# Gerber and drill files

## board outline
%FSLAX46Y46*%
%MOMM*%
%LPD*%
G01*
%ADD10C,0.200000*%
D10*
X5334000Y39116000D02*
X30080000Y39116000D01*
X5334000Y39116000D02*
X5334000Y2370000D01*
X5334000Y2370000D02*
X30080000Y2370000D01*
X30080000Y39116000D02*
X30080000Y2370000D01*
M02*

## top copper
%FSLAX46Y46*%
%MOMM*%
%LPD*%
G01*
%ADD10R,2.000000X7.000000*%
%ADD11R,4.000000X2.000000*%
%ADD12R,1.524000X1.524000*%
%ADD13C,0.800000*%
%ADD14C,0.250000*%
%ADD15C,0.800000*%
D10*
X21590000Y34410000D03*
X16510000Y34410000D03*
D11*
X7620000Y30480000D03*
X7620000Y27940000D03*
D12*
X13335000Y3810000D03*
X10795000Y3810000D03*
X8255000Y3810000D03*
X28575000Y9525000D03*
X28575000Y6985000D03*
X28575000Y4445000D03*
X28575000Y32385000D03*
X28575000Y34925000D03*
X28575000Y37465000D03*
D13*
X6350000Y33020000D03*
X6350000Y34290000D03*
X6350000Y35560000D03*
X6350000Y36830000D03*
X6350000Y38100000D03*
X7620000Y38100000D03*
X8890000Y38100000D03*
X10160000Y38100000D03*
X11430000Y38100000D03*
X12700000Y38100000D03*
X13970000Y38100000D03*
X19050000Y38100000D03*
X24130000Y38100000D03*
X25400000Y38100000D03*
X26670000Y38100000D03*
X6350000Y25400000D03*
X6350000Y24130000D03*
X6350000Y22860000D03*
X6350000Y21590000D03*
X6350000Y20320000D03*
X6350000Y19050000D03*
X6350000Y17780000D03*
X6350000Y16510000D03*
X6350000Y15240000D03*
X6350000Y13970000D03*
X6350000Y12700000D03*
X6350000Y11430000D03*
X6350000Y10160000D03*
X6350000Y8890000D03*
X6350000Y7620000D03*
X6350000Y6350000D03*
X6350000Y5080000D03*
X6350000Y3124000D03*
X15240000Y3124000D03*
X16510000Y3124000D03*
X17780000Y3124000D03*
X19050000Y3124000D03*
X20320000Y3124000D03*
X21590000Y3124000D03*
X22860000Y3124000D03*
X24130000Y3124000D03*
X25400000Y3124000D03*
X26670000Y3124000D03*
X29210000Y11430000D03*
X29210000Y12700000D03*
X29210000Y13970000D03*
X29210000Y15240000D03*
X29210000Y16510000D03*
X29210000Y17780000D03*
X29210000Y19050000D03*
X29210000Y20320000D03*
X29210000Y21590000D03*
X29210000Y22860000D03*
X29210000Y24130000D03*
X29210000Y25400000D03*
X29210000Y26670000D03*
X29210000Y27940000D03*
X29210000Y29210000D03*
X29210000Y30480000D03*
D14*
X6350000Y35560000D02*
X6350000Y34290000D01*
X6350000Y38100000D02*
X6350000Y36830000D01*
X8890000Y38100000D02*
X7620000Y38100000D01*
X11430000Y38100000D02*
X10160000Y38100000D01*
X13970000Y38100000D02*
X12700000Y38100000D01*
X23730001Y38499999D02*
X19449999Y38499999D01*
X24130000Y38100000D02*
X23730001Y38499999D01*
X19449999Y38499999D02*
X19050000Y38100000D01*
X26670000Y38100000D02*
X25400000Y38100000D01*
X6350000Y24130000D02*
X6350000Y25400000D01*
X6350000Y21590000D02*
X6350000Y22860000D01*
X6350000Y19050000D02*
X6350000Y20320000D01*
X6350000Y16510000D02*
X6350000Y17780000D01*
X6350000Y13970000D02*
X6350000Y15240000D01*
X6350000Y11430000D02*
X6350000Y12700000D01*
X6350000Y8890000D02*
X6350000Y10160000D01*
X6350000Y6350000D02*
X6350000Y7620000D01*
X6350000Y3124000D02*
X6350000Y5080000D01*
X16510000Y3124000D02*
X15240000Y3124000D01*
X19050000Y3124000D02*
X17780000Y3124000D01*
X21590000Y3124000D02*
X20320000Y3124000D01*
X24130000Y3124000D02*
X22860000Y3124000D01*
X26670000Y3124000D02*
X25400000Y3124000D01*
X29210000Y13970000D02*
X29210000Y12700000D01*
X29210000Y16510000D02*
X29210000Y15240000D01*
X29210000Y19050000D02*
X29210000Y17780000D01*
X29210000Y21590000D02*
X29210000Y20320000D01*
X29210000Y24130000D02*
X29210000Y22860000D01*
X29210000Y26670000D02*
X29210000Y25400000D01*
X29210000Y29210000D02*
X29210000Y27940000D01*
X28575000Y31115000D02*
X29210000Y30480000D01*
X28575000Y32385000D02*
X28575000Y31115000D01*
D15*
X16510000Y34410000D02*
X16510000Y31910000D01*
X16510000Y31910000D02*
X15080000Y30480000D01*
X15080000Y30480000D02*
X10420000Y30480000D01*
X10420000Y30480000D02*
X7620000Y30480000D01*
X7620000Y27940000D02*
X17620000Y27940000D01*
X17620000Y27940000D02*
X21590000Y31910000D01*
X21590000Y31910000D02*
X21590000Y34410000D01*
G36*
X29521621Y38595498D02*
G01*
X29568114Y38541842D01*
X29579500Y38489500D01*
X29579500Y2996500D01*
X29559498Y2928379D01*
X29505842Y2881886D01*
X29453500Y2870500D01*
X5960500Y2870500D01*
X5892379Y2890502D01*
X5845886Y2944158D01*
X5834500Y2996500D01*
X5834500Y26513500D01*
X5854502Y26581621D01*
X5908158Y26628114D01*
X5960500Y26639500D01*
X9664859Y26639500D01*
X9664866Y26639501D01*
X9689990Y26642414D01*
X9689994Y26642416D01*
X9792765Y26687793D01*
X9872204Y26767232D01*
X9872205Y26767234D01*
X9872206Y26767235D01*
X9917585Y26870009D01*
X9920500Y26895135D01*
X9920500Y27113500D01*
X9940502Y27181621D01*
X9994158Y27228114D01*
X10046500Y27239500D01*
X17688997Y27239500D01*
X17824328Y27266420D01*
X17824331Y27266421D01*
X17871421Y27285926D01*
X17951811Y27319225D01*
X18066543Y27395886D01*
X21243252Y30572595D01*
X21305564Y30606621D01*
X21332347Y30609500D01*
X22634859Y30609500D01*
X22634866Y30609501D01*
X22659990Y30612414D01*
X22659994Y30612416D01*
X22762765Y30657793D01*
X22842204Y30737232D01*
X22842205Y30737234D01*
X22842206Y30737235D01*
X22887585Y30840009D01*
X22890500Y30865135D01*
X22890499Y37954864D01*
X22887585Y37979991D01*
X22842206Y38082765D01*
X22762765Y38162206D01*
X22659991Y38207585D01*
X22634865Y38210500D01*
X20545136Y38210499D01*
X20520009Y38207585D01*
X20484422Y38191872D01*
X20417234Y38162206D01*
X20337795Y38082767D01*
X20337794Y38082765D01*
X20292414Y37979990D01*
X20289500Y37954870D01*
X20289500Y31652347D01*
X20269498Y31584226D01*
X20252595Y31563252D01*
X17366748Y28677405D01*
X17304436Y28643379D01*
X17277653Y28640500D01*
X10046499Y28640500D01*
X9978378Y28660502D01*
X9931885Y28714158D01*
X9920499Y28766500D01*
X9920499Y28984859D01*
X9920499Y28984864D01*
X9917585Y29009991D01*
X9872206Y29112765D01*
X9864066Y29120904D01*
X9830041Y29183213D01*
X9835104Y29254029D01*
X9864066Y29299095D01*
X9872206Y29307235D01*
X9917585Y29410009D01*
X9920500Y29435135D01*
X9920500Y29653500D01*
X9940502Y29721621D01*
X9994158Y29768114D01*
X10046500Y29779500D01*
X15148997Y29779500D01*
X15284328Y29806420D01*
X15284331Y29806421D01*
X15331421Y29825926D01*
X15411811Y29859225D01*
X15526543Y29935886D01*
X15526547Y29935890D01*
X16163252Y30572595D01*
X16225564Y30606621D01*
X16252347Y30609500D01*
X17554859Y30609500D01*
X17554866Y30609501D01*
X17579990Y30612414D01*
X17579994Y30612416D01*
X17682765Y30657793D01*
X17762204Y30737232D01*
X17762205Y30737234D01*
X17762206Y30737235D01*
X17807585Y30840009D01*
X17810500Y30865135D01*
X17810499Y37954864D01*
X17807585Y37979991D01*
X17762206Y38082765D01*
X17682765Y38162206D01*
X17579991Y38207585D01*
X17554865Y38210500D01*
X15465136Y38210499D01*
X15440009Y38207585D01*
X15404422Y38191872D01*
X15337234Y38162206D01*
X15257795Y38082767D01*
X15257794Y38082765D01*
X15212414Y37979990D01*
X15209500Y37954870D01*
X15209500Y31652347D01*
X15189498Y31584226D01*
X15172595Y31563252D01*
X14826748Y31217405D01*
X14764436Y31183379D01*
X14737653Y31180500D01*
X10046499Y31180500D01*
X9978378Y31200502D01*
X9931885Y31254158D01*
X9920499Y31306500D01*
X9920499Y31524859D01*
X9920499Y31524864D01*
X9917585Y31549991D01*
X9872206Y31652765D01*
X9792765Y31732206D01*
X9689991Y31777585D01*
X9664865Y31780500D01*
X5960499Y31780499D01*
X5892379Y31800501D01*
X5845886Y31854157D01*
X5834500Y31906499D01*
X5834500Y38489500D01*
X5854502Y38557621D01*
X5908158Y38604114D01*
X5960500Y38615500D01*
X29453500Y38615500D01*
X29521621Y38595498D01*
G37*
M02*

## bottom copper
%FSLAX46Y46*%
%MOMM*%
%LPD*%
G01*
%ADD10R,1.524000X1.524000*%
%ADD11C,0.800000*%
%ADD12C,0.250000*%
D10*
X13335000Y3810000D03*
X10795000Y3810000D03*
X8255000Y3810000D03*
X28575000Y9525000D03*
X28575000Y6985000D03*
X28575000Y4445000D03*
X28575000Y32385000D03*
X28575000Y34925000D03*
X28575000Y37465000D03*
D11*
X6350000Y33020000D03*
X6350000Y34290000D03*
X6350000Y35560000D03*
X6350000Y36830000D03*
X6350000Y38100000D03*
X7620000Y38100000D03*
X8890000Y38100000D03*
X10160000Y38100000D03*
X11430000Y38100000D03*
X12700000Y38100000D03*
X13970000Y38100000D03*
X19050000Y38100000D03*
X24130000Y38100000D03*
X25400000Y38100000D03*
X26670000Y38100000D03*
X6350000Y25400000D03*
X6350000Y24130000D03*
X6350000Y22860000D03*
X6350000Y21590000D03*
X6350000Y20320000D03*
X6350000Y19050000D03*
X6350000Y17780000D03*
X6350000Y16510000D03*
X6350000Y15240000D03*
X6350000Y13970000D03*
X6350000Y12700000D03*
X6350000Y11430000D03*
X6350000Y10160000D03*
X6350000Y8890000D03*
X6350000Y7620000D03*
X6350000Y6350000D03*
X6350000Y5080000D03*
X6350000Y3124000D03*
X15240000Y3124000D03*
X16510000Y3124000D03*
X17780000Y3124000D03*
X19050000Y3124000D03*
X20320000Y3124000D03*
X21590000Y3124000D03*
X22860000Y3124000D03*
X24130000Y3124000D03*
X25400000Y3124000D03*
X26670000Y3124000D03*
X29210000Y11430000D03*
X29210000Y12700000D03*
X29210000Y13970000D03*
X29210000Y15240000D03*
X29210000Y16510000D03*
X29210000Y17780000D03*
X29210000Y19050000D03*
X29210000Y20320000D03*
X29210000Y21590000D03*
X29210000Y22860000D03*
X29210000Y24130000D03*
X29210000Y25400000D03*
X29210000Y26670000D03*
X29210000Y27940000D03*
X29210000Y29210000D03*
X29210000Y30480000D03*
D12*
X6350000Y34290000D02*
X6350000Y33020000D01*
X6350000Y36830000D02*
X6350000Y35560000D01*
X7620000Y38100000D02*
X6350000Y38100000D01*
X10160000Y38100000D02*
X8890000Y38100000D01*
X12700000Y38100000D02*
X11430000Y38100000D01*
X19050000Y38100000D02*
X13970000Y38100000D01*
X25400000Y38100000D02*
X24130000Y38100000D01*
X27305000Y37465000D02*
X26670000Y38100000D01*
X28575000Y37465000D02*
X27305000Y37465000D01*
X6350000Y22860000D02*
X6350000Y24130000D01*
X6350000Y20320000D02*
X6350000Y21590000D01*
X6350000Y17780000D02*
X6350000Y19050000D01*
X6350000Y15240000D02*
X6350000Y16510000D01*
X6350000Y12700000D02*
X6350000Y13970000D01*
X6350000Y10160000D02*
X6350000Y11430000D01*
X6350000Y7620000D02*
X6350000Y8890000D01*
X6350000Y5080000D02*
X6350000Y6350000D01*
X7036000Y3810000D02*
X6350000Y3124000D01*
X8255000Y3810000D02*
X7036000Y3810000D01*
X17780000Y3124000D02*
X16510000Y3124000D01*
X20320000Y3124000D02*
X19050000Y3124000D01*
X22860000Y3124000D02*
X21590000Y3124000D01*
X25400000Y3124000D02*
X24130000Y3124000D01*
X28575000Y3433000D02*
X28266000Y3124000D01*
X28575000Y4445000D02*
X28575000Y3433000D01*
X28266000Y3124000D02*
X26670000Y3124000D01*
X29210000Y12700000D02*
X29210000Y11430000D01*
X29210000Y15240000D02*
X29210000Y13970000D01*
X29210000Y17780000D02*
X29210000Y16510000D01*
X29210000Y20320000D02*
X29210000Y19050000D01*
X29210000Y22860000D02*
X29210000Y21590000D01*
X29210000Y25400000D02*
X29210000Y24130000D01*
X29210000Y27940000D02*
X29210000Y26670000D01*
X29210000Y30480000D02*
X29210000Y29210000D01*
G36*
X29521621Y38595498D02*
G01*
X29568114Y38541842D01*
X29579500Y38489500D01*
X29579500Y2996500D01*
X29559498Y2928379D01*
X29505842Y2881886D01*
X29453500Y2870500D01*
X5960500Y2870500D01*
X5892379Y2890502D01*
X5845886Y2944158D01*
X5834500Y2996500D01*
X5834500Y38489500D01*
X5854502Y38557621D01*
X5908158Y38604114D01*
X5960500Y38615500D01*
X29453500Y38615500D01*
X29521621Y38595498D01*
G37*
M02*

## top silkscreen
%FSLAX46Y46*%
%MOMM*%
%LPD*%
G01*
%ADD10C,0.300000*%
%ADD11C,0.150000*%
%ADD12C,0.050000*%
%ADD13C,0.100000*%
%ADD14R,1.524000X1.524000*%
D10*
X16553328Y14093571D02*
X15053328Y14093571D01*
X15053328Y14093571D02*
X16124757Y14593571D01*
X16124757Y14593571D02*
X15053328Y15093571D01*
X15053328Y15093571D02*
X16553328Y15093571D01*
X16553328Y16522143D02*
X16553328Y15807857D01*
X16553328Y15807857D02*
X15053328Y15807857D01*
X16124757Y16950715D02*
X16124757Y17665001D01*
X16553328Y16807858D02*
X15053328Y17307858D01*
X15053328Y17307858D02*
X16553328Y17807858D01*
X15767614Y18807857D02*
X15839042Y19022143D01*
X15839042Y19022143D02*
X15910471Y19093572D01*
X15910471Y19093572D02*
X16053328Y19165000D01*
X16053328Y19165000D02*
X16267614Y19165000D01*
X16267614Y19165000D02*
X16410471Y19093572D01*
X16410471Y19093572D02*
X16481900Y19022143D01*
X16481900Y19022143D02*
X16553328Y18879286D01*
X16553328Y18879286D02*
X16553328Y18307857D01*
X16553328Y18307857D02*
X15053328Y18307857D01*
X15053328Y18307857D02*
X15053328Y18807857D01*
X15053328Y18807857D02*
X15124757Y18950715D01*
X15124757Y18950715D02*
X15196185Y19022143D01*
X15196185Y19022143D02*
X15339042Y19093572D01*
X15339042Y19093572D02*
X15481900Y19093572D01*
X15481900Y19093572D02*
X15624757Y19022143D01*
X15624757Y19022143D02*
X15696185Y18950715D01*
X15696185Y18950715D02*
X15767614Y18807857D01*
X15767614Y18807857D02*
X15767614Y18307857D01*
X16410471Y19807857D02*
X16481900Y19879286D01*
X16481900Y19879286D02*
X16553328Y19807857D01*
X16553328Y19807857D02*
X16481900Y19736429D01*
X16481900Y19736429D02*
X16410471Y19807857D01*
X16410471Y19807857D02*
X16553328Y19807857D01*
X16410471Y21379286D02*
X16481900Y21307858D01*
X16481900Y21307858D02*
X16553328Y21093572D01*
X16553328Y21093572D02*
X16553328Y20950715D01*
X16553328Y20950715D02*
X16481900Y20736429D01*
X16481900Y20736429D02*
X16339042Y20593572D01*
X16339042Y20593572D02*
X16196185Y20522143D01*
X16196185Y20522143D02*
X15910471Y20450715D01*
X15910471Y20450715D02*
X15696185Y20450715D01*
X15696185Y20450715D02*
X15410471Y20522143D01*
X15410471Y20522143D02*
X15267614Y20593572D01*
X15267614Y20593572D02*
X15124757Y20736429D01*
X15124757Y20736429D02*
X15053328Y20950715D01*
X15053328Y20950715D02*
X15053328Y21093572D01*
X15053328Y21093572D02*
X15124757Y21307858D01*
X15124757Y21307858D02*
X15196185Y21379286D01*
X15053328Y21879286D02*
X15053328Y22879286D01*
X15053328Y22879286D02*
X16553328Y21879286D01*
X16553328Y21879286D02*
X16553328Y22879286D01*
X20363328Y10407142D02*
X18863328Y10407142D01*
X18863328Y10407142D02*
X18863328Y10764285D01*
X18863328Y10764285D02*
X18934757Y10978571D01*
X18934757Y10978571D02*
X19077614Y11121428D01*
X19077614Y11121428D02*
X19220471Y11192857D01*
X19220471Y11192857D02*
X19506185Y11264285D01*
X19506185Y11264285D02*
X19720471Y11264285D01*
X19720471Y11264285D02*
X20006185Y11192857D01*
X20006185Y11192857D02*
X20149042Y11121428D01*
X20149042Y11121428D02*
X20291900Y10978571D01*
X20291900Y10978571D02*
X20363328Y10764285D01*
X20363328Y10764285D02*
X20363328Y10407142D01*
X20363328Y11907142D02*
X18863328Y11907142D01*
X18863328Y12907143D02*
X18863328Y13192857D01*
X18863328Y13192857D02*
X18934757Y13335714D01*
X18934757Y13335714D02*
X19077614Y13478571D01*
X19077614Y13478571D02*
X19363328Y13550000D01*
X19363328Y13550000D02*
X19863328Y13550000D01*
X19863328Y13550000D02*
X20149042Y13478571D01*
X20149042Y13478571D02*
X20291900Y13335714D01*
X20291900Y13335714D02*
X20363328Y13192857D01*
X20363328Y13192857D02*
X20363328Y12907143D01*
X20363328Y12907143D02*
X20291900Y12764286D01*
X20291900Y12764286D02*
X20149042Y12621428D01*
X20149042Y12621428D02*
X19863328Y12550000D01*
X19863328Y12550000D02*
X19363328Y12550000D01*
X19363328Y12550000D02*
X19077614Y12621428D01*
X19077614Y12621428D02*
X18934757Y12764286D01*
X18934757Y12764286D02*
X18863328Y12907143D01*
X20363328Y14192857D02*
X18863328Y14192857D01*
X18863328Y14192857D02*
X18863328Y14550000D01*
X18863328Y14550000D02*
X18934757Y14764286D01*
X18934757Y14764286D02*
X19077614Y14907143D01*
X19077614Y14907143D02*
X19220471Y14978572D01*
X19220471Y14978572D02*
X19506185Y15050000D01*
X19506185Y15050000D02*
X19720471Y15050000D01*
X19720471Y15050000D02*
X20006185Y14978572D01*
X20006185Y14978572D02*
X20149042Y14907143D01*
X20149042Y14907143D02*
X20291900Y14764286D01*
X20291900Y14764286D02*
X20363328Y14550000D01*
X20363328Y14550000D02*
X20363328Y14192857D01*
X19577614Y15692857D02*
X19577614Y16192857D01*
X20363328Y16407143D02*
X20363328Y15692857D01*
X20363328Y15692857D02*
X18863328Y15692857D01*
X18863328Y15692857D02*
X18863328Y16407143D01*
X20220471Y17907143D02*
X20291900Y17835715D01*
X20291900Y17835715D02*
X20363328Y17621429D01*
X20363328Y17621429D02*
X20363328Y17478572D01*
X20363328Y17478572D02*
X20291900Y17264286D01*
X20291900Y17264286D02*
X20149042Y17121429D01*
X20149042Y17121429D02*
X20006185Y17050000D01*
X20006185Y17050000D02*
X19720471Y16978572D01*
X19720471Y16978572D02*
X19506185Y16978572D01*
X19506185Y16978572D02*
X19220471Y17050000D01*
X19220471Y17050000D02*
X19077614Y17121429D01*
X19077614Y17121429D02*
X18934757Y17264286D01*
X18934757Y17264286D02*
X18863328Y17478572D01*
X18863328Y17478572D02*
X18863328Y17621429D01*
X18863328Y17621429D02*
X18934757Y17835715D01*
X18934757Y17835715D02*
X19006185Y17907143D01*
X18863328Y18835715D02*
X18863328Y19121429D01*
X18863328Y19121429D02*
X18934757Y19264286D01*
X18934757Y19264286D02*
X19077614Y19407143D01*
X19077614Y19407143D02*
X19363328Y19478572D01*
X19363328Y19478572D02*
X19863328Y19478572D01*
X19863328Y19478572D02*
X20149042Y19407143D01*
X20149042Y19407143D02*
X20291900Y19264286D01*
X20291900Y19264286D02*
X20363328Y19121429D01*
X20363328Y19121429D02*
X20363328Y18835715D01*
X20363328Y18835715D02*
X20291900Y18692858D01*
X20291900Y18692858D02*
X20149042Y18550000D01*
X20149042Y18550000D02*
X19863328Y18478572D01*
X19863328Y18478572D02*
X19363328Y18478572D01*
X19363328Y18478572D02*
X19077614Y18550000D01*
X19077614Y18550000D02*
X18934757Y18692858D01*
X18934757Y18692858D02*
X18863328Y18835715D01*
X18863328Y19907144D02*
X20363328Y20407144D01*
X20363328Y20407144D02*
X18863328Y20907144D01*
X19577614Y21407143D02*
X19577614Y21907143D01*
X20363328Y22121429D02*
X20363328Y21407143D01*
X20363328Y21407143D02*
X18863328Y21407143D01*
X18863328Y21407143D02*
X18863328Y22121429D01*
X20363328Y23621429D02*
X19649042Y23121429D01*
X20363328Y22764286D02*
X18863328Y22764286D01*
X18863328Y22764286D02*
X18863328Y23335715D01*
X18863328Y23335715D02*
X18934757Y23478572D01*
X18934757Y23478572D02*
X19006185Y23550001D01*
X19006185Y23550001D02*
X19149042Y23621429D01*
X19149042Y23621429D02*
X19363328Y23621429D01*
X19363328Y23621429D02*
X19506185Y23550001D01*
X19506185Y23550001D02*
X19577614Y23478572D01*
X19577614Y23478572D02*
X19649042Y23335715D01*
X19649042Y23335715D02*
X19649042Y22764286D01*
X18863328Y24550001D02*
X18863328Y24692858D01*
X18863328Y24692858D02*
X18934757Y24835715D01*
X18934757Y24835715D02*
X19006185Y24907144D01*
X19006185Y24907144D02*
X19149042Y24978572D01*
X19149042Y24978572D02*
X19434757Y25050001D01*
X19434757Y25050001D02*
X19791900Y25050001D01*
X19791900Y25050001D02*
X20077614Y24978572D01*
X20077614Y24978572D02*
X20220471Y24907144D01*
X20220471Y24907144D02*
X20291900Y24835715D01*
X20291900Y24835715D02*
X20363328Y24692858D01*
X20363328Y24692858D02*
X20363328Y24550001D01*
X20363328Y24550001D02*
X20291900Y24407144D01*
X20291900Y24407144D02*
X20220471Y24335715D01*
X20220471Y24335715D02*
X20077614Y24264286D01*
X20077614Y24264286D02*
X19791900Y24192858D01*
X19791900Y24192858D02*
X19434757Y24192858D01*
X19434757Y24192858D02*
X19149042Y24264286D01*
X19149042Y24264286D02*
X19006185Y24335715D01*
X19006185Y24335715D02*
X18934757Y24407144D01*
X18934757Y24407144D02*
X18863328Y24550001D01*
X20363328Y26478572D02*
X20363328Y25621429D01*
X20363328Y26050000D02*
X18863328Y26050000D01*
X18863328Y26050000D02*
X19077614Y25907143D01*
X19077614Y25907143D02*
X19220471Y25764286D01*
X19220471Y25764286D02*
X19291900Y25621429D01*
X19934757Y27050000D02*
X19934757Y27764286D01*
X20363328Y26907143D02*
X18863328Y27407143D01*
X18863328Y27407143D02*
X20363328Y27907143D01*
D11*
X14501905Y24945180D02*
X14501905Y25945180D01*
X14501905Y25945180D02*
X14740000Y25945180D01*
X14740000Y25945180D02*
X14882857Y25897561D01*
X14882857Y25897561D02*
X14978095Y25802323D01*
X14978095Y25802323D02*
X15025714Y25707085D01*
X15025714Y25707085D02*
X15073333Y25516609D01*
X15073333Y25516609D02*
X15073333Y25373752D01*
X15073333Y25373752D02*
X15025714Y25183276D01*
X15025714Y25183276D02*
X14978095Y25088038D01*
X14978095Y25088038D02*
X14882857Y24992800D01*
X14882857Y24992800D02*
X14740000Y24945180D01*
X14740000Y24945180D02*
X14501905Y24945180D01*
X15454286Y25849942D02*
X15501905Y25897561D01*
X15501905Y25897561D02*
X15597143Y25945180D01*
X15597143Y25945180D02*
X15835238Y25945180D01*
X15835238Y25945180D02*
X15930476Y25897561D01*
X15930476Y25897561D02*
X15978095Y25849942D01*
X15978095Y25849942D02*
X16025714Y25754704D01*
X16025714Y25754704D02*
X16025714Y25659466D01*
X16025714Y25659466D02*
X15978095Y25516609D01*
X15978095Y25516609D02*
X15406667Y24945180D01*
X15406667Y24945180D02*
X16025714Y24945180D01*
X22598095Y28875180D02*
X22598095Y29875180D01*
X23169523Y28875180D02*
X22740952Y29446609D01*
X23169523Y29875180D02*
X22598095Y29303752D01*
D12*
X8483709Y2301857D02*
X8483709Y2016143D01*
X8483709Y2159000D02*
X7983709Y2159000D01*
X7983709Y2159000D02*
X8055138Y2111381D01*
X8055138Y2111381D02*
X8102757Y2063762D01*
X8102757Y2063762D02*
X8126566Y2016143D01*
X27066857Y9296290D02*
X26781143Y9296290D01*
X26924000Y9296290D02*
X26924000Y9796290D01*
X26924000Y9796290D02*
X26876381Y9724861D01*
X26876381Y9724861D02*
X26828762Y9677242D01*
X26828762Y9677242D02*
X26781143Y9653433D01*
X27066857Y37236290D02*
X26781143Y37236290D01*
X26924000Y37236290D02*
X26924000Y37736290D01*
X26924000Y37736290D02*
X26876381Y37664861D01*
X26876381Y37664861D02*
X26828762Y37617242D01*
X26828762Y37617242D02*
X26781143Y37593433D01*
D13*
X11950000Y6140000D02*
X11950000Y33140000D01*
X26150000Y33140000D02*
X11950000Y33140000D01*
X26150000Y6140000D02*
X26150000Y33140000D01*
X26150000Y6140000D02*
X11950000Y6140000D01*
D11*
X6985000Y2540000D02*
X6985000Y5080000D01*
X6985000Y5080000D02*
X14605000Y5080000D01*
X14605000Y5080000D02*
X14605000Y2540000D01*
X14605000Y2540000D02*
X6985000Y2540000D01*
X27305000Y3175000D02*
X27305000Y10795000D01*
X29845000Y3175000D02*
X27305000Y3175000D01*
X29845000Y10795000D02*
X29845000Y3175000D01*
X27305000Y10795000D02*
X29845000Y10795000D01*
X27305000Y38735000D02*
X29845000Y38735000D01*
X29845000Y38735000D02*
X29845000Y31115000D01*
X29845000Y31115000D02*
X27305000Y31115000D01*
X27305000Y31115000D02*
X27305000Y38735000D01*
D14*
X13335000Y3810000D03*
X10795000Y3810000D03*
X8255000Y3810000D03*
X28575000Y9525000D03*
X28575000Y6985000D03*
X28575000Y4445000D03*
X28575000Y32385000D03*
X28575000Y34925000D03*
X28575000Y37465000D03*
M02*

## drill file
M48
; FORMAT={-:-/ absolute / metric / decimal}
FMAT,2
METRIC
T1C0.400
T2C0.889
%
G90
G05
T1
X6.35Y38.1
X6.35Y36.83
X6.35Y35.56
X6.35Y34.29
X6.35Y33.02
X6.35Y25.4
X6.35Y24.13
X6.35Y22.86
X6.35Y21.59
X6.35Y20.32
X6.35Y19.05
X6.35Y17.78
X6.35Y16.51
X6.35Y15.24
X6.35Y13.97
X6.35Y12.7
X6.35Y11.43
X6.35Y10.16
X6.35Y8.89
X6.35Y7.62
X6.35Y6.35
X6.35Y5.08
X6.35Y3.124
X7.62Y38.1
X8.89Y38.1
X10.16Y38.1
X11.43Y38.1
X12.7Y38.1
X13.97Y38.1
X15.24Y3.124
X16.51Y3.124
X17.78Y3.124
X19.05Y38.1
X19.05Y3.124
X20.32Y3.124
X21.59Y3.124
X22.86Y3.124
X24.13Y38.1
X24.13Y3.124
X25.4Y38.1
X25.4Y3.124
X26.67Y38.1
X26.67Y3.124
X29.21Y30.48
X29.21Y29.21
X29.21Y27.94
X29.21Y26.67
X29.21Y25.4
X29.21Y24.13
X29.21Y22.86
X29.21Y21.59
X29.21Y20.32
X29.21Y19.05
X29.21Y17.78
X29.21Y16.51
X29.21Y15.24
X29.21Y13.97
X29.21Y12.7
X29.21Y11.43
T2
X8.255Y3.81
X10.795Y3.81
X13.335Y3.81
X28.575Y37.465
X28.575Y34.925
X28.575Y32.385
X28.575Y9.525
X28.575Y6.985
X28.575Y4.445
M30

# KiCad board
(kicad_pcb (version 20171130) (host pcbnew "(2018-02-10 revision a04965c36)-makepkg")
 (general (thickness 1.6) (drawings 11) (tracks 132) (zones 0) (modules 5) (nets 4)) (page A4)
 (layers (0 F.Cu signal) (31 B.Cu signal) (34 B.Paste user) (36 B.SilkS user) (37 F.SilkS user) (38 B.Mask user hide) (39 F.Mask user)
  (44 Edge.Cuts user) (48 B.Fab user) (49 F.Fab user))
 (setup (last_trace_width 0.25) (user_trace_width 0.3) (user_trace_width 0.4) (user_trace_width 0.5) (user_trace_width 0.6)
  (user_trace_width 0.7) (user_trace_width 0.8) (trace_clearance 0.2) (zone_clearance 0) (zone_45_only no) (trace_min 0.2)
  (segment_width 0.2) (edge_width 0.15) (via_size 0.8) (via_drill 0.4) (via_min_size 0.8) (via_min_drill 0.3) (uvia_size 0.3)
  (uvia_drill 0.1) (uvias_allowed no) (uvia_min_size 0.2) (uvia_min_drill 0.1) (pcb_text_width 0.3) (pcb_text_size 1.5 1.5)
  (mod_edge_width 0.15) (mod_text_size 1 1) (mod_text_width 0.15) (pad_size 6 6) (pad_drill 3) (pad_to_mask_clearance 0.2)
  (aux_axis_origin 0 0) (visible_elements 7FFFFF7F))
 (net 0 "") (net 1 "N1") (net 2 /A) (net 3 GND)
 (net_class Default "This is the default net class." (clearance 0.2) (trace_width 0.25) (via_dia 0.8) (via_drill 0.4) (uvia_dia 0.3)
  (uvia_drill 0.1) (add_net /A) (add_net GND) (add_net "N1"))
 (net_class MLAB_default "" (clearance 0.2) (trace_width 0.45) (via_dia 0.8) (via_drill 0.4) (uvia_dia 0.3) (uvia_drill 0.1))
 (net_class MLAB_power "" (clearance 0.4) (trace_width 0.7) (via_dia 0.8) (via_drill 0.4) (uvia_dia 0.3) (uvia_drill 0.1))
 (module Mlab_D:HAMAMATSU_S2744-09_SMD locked (layer F.Cu) (at 19.05 -5.2 270)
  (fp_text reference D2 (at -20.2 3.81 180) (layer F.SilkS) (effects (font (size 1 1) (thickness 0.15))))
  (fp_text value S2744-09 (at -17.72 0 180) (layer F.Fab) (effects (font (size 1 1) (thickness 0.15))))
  (fp_line (start -0.94 7.1) (end -27.94 7.1) (layer F.SilkS) (width 0.1))
  (fp_line (start -27.94 -7.1) (end -27.94 7.1) (layer F.SilkS) (width 0.1))
  (fp_line (start -0.94 -7.1) (end -27.94 -7.1) (layer F.SilkS) (width 0.1))
  (fp_line (start -0.94 -7.1) (end -0.94 7.1) (layer F.SilkS) (width 0.1))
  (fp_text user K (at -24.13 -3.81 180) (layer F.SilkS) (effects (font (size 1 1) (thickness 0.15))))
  (pad 1 smd rect (at -29.21 -2.54 270) (size 7 2) (layers F.Cu F.Mask) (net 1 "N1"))
  (pad 2 smd rect (at -29.21 2.54 270) (size 7 2) (layers F.Cu F.Mask) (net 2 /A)))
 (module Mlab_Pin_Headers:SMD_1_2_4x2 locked (layer F.Cu) (at 7.62 -27.94 180)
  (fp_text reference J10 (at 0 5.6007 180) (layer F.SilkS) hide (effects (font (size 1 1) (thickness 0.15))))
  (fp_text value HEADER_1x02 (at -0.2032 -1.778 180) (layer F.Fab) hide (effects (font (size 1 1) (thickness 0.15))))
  (pad 2 smd rect (at 0 2.54 180) (size 4 2) (layers F.Cu F.Mask) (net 2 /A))
  (pad 1 smd rect (at 0 0 180) (size 4 2) (layers F.Cu F.Mask) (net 1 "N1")))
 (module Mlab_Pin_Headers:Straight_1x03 (layer F.Cu) (at 10.795 -3.81 90)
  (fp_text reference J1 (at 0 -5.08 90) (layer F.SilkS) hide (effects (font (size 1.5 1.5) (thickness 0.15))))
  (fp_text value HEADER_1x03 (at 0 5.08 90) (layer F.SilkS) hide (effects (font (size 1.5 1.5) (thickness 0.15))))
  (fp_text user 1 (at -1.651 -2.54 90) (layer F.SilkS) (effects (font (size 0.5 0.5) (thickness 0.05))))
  (fp_line (start -1.27 -3.81) (end 1.27 -3.81) (layer F.SilkS) (width 0.15))
  (fp_line (start 1.27 -3.81) (end 1.27 3.81) (layer F.SilkS) (width 0.15))
  (fp_line (start 1.27 3.81) (end -1.27 3.81) (layer F.SilkS) (width 0.15))
  (fp_line (start -1.27 3.81) (end -1.27 -3.81) (layer F.SilkS) (width 0.15))
  (pad 3 thru_hole rect (at 0 2.54 90) (size 1.524 1.524) (drill 0.889) (layers *.Cu *.Mask F.SilkS) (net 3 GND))
  (pad 2 thru_hole rect (at 0 0 90) (size 1.524 1.524) (drill 0.889) (layers *.Cu *.Mask F.SilkS) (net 3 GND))
  (pad 1 thru_hole rect (at 0 -2.54 90) (size 1.524 1.524) (drill 0.889) (layers *.Cu *.Mask F.SilkS) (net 3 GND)))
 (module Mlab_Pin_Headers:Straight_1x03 (layer F.Cu) (at 28.575 -6.985)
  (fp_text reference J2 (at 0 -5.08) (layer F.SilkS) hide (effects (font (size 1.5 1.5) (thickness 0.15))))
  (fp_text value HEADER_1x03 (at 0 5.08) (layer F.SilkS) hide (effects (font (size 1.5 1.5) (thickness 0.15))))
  (fp_line (start -1.27 3.81) (end -1.27 -3.81) (layer F.SilkS) (width 0.15))
  (fp_line (start 1.27 3.81) (end -1.27 3.81) (layer F.SilkS) (width 0.15))
  (fp_line (start 1.27 -3.81) (end 1.27 3.81) (layer F.SilkS) (width 0.15))
  (fp_line (start -1.27 -3.81) (end 1.27 -3.81) (layer F.SilkS) (width 0.15))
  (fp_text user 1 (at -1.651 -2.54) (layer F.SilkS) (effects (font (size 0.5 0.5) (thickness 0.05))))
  (pad 1 thru_hole rect (at 0 -2.54) (size 1.524 1.524) (drill 0.889) (layers *.Cu *.Mask F.SilkS) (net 3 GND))
  (pad 2 thru_hole rect (at 0 0) (size 1.524 1.524) (drill 0.889) (layers *.Cu *.Mask F.SilkS) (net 3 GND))
  (pad 3 thru_hole rect (at 0 2.54) (size 1.524 1.524) (drill 0.889) (layers *.Cu *.Mask F.SilkS) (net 3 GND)))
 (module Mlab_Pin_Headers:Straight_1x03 (layer F.Cu) (at 28.575 -34.925)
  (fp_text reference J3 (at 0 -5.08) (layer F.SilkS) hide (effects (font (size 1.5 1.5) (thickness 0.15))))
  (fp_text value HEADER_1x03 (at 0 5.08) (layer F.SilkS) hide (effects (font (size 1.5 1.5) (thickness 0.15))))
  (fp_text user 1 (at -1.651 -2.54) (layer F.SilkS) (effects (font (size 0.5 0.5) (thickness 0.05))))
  (fp_line (start -1.27 -3.81) (end 1.27 -3.81) (layer F.SilkS) (width 0.15))
  (fp_line (start 1.27 -3.81) (end 1.27 3.81) (layer F.SilkS) (width 0.15))
  (fp_line (start 1.27 3.81) (end -1.27 3.81) (layer F.SilkS) (width 0.15))
  (fp_line (start -1.27 3.81) (end -1.27 -3.81) (layer F.SilkS) (width 0.15))
  (pad 3 thru_hole rect (at 0 2.54) (size 1.524 1.524) (drill 0.889) (layers *.Cu *.Mask F.SilkS) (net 3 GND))
  (pad 2 thru_hole rect (at 0 0) (size 1.524 1.524) (drill 0.889) (layers *.Cu *.Mask F.SilkS) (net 3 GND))
  (pad 1 thru_hole rect (at 0 -2.54) (size 1.524 1.524) (drill 0.889) (layers *.Cu *.Mask F.SilkS) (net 3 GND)))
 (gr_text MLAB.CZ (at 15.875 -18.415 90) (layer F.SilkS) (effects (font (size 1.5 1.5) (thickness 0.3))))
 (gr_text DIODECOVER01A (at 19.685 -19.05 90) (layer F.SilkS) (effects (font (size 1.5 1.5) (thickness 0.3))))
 (gr_line (start 5.334 -39.116) (end 30.08 -39.116) (layer Edge.Cuts) (width 0.2))
 (gr_line (start 5.334 -39.116) (end 5.334 -2.37) (layer Edge.Cuts) (width 0.2))
 (gr_line (start 5.334 -2.37) (end 30.08 -2.37) (layer Edge.Cuts) (width 0.2))
 (gr_line (start 30.08 -39.116) (end 30.08 -2.37) (layer Edge.Cuts) (width 0.2))
 (segment (start 6.35 -34.29) (end 6.35 -33.02) (width 0.25) (layer B.Cu) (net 3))
 (via (at 6.35 -33.02) (size 0.8) (drill 0.4) (layers F.Cu B.Cu) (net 3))
 (segment (start 6.35 -35.56) (end 6.35 -34.29) (width 0.25) (layer F.Cu) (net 3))
 (via (at 6.35 -34.29) (size 0.8) (drill 0.4) (layers F.Cu B.Cu) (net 3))
 (segment (start 6.35 -36.83) (end 6.35 -35.56) (width 0.25) (layer B.Cu) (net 3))
 (via (at 6.35 -35.56) (size 0.8) (drill 0.4) (layers F.Cu B.Cu) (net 3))
 (segment (start 6.35 -38.1) (end 6.35 -36.83) (width 0.25) (layer F.Cu) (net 3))
 (via (at 6.35 -36.83) (size 0.8) (drill 0.4) (layers F.Cu B.Cu) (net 3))
 (segment (start 7.62 -38.1) (end 6.35 -38.1) (width 0.25) (layer B.Cu) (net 3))
 (via (at 6.35 -38.1) (size 0.8) (drill 0.4) (layers F.Cu B.Cu) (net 3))
 (segment (start 8.89 -38.1) (end 7.62 -38.1) (width 0.25) (layer F.Cu) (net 3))
 (via (at 7.62 -38.1) (size 0.8) (drill 0.4) (layers F.Cu B.Cu) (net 3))
 (segment (start 10.16 -38.1) (end 8.89 -38.1) (width 0.25) (layer B.Cu) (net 3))
 (via (at 8.89 -38.1) (size 0.8) (drill 0.4) (layers F.Cu B.Cu) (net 3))
 (segment (start 11.43 -38.1) (end 10.16 -38.1) (width 0.25) (layer F.Cu) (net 3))
 (via (at 10.16 -38.1) (size 0.8) (drill 0.4) (layers F.Cu B.Cu) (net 3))
 (segment (start 12.7 -38.1) (end 11.43 -38.1) (width 0.25) (layer B.Cu) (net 3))
 (via (at 11.43 -38.1) (size 0.8) (drill 0.4) (layers F.Cu B.Cu) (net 3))
 (segment (start 13.97 -38.1) (end 12.7 -38.1) (width 0.25) (layer F.Cu) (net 3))
 (via (at 12.7 -38.1) (size 0.8) (drill 0.4) (layers F.Cu B.Cu) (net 3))
 (segment (start 19.05 -38.1) (end 13.97 -38.1) (width 0.25) (layer B.Cu) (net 3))
 (via (at 13.97 -38.1) (size 0.8) (drill 0.4) (layers F.Cu B.Cu) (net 3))
 (segment (start 23.730001 -38.499999) (end 19.449999 -38.499999) (width 0.25) (layer F.Cu) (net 3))
 (segment (start 24.13 -38.1) (end 23.730001 -38.499999) (width 0.25) (layer F.Cu) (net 3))
 (segment (start 19.449999 -38.499999) (end 19.05 -38.1) (width 0.25) (layer F.Cu) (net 3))
 (via (at 19.05 -38.1) (size 0.8) (drill 0.4) (layers F.Cu B.Cu) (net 3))
 (segment (start 25.4 -38.1) (end 24.13 -38.1) (width 0.25) (layer B.Cu) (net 3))
 (via (at 24.13 -38.1) (size 0.8) (drill 0.4) (layers F.Cu B.Cu) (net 3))
 (segment (start 26.67 -38.1) (end 25.4 -38.1) (width 0.25) (layer F.Cu) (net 3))
 (via (at 25.4 -38.1) (size 0.8) (drill 0.4) (layers F.Cu B.Cu) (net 3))
 (segment (start 27.305 -37.465) (end 26.67 -38.1) (width 0.25) (layer B.Cu) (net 3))
 (segment (start 28.575 -37.465) (end 27.305 -37.465) (width 0.25) (layer B.Cu) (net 3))
 (via (at 26.67 -38.1) (size 0.8) (drill 0.4) (layers F.Cu B.Cu) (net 3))
 (segment (start 6.35 -24.13) (end 6.35 -25.4) (width 0.25) (layer F.Cu) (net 3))
 (via (at 6.35 -25.4) (size 0.8) (drill 0.4) (layers F.Cu B.Cu) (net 3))
 (segment (start 6.35 -22.86) (end 6.35 -24.13) (width 0.25) (layer B.Cu) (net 3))
 (via (at 6.35 -24.13) (size 0.8) (drill 0.4) (layers F.Cu B.Cu) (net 3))
 (segment (start 6.35 -21.59) (end 6.35 -22.86) (width 0.25) (layer F.Cu) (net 3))
 (via (at 6.35 -22.86) (size 0.8) (drill 0.4) (layers F.Cu B.Cu) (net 3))
 (segment (start 6.35 -20.32) (end 6.35 -21.59) (width 0.25) (layer B.Cu) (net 3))
 (via (at 6.35 -21.59) (size 0.8) (drill 0.4) (layers F.Cu B.Cu) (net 3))
 (segment (start 6.35 -19.05) (end 6.35 -20.32) (width 0.25) (layer F.Cu) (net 3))
 (via (at 6.35 -20.32) (size 0.8) (drill 0.4) (layers F.Cu B.Cu) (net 3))
 (segment (start 6.35 -17.78) (end 6.35 -19.05) (width 0.25) (layer B.Cu) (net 3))
 (via (at 6.35 -19.05) (size 0.8) (drill 0.4) (layers F.Cu B.Cu) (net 3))
 (segment (start 6.35 -16.51) (end 6.35 -17.78) (width 0.25) (layer F.Cu) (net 3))
 (via (at 6.35 -17.78) (size 0.8) (drill 0.4) (layers F.Cu B.Cu) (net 3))
 (segment (start 6.35 -15.24) (end 6.35 -16.51) (width 0.25) (layer B.Cu) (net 3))
 (via (at 6.35 -16.51) (size 0.8) (drill 0.4) (layers F.Cu B.Cu) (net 3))
 (segment (start 6.35 -13.97) (end 6.35 -15.24) (width 0.25) (layer F.Cu) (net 3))
 (via (at 6.35 -15.24) (size 0.8) (drill 0.4) (layers F.Cu B.Cu) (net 3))
 (segment (start 6.35 -12.7) (end 6.35 -13.97) (width 0.25) (layer B.Cu) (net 3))
 (via (at 6.35 -13.97) (size 0.8) (drill 0.4) (layers F.Cu B.Cu) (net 3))
 (segment (start 6.35 -11.43) (end 6.35 -12.7) (width 0.25) (layer F.Cu) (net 3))
 (via (at 6.35 -12.7) (size 0.8) (drill 0.4) (layers F.Cu B.Cu) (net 3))
 (segment (start 6.35 -10.16) (end 6.35 -11.43) (width 0.25) (layer B.Cu) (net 3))
 (via (at 6.35 -11.43) (size 0.8) (drill 0.4) (layers F.Cu B.Cu) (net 3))
 (segment (start 6.35 -8.89) (end 6.35 -10.16) (width 0.25) (layer F.Cu) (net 3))
 (via (at 6.35 -10.16) (size 0.8) (drill 0.4) (layers F.Cu B.Cu) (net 3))
 (segment (start 6.35 -7.62) (end 6.35 -8.89) (width 0.25) (layer B.Cu) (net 3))
 (via (at 6.35 -8.89) (size 0.8) (drill 0.4) (layers F.Cu B.Cu) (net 3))
 (segment (start 6.35 -6.35) (end 6.35 -7.62) (width 0.25) (layer F.Cu) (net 3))
 (via (at 6.35 -7.62) (size 0.8) (drill 0.4) (layers F.Cu B.Cu) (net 3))
 (segment (start 6.35 -5.08) (end 6.35 -6.35) (width 0.25) (layer B.Cu) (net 3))
 (via (at 6.35 -6.35) (size 0.8) (drill 0.4) (layers F.Cu B.Cu) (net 3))
 (segment (start 6.35 -3.124) (end 6.35 -5.08) (width 0.25) (layer F.Cu) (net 3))
 (via (at 6.35 -5.08) (size 0.8) (drill 0.4) (layers F.Cu B.Cu) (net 3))
 (segment (start 7.036 -3.81) (end 6.35 -3.124) (width 0.25) (layer B.Cu) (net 3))
 (segment (start 8.255 -3.81) (end 7.036 -3.81) (width 0.25) (layer B.Cu) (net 3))
 (via (at 6.35 -3.124) (size 0.8) (drill 0.4) (layers F.Cu B.Cu) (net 3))
 (segment (start 16.51 -3.124) (end 15.24 -3.124) (width 0.25) (layer F.Cu) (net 3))
 (via (at 15.24 -3.124) (size 0.8) (drill 0.4) (layers F.Cu B.Cu) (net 3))
 (segment (start 17.78 -3.124) (end 16.51 -3.124) (width 0.25) (layer B.Cu) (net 3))
 (via (at 16.51 -3.124) (size 0.8) (drill 0.4) (layers F.Cu B.Cu) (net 3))
 (segment (start 19.05 -3.124) (end 17.78 -3.124) (width 0.25) (layer F.Cu) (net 3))
 (via (at 17.78 -3.124) (size 0.8) (drill 0.4) (layers F.Cu B.Cu) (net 3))
 (segment (start 20.32 -3.124) (end 19.05 -3.124) (width 0.25) (layer B.Cu) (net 3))
 (via (at 19.05 -3.124) (size 0.8) (drill 0.4) (layers F.Cu B.Cu) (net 3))
 (segment (start 21.59 -3.124) (end 20.32 -3.124) (width 0.25) (layer F.Cu) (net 3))
 (via (at 20.32 -3.124) (size 0.8) (drill 0.4) (layers F.Cu B.Cu) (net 3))
 (segment (start 22.86 -3.124) (end 21.59 -3.124) (width 0.25) (layer B.Cu) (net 3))
 (via (at 21.59 -3.124) (size 0.8) (drill 0.4) (layers F.Cu B.Cu) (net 3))
 (segment (start 24.13 -3.124) (end 22.86 -3.124) (width 0.25) (layer F.Cu) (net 3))
 (via (at 22.86 -3.124) (size 0.8) (drill 0.4) (layers F.Cu B.Cu) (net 3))
 (segment (start 25.4 -3.124) (end 24.13 -3.124) (width 0.25) (layer B.Cu) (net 3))
 (via (at 24.13 -3.124) (size 0.8) (drill 0.4) (layers F.Cu B.Cu) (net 3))
 (segment (start 26.67 -3.124) (end 25.4 -3.124) (width 0.25) (layer F.Cu) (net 3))
 (via (at 25.4 -3.124) (size 0.8) (drill 0.4) (layers F.Cu B.Cu) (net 3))
 (segment (start 28.575 -3.433) (end 28.266 -3.124) (width 0.25) (layer B.Cu) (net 3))
 (segment (start 28.575 -4.445) (end 28.575 -3.433) (width 0.25) (layer B.Cu) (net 3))
 (segment (start 28.266 -3.124) (end 26.67 -3.124) (width 0.25) (layer B.Cu) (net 3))
 (via (at 26.67 -3.124) (size 0.8) (drill 0.4) (layers F.Cu B.Cu) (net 3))
 (via (at 29.21 -11.43) (size 0.8) (drill 0.4) (layers F.Cu B.Cu) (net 3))
 (segment (start 29.21 -12.7) (end 29.21 -11.43) (width 0.25) (layer B.Cu) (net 3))
 (segment (start 29.21 -13.97) (end 29.21 -12.7) (width 0.25) (layer F.Cu) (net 3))
 (via (at 29.21 -12.7) (size 0.8) (drill 0.4) (layers F.Cu B.Cu) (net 3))
 (segment (start 29.21 -15.24) (end 29.21 -13.97) (width 0.25) (layer B.Cu) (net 3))
 (via (at 29.21 -13.97) (size 0.8) (drill 0.4) (layers F.Cu B.Cu) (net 3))
 (segment (start 29.21 -16.51) (end 29.21 -15.24) (width 0.25) (layer F.Cu) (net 3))
 (via (at 29.21 -15.24) (size 0.8) (drill 0.4) (layers F.Cu B.Cu) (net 3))
 (segment (start 29.21 -17.78) (end 29.21 -16.51) (width 0.25) (layer B.Cu) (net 3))
 (via (at 29.21 -16.51) (size 0.8) (drill 0.4) (layers F.Cu B.Cu) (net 3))
 (segment (start 29.21 -19.05) (end 29.21 -17.78) (width 0.25) (layer F.Cu) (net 3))
 (via (at 29.21 -17.78) (size 0.8) (drill 0.4) (layers F.Cu B.Cu) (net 3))
 (segment (start 29.21 -20.32) (end 29.21 -19.05) (width 0.25) (layer B.Cu) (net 3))
 (via (at 29.21 -19.05) (size 0.8) (drill 0.4) (layers F.Cu B.Cu) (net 3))
 (segment (start 29.21 -21.59) (end 29.21 -20.32) (width 0.25) (layer F.Cu) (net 3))
 (via (at 29.21 -20.32) (size 0.8) (drill 0.4) (layers F.Cu B.Cu) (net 3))
 (segment (start 29.21 -22.86) (end 29.21 -21.59) (width 0.25) (layer B.Cu) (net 3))
 (via (at 29.21 -21.59) (size 0.8) (drill 0.4) (layers F.Cu B.Cu) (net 3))
 (segment (start 29.21 -24.13) (end 29.21 -22.86) (width 0.25) (layer F.Cu) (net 3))
 (via (at 29.21 -22.86) (size 0.8) (drill 0.4) (layers F.Cu B.Cu) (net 3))
 (segment (start 29.21 -25.4) (end 29.21 -24.13) (width 0.25) (layer B.Cu) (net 3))
 (via (at 29.21 -24.13) (size 0.8) (drill 0.4) (layers F.Cu B.Cu) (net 3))
 (segment (start 29.21 -26.67) (end 29.21 -25.4) (width 0.25) (layer F.Cu) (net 3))
 (via (at 29.21 -25.4) (size 0.8) (drill 0.4) (layers F.Cu B.Cu) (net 3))
 (segment (start 29.21 -27.94) (end 29.21 -26.67) (width 0.25) (layer B.Cu) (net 3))
 (via (at 29.21 -26.67) (size 0.8) (drill 0.4) (layers F.Cu B.Cu) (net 3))
 (segment (start 29.21 -29.21) (end 29.21 -27.94) (width 0.25) (layer F.Cu) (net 3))
 (via (at 29.21 -27.94) (size 0.8) (drill 0.4) (layers F.Cu B.Cu) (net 3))
 (segment (start 29.21 -30.48) (end 29.21 -29.21) (width 0.25) (layer B.Cu) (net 3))
 (via (at 29.21 -29.21) (size 0.8) (drill 0.4) (layers F.Cu B.Cu) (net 3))
 (segment (start 28.575 -31.115) (end 29.21 -30.48) (width 0.25) (layer F.Cu) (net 3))
 (segment (start 28.575 -32.385) (end 28.575 -31.115) (width 0.25) (layer F.Cu) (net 3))
 (via (at 29.21 -30.48) (size 0.8) (drill 0.4) (layers F.Cu B.Cu) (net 3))
 (segment (start 16.51 -34.41) (end 16.51 -31.91) (width 0.8) (layer F.Cu) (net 2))
 (segment (start 16.51 -31.91) (end 15.08 -30.48) (width 0.8) (layer F.Cu) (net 2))
 (segment (start 15.08 -30.48) (end 10.42 -30.48) (width 0.8) (layer F.Cu) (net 2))
 (segment (start 10.42 -30.48) (end 7.62 -30.48) (width 0.8) (layer F.Cu) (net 2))
 (segment (start 7.62 -27.94) (end 17.62 -27.94) (width 0.8) (layer F.Cu) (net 1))
 (segment (start 17.62 -27.94) (end 21.59 -31.91) (width 0.8) (layer F.Cu) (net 1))
 (segment (start 21.59 -31.91) (end 21.59 -34.41) (width 0.8) (layer F.Cu) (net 1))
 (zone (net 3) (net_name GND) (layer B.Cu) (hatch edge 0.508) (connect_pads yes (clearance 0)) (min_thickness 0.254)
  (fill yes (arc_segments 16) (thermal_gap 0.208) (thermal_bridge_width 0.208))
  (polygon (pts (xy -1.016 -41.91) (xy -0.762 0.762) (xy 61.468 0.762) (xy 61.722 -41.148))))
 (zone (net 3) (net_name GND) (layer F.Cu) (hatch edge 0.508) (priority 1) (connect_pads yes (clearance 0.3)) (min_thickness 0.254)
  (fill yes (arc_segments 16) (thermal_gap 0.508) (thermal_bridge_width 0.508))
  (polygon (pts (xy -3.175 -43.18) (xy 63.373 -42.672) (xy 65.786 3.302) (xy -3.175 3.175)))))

